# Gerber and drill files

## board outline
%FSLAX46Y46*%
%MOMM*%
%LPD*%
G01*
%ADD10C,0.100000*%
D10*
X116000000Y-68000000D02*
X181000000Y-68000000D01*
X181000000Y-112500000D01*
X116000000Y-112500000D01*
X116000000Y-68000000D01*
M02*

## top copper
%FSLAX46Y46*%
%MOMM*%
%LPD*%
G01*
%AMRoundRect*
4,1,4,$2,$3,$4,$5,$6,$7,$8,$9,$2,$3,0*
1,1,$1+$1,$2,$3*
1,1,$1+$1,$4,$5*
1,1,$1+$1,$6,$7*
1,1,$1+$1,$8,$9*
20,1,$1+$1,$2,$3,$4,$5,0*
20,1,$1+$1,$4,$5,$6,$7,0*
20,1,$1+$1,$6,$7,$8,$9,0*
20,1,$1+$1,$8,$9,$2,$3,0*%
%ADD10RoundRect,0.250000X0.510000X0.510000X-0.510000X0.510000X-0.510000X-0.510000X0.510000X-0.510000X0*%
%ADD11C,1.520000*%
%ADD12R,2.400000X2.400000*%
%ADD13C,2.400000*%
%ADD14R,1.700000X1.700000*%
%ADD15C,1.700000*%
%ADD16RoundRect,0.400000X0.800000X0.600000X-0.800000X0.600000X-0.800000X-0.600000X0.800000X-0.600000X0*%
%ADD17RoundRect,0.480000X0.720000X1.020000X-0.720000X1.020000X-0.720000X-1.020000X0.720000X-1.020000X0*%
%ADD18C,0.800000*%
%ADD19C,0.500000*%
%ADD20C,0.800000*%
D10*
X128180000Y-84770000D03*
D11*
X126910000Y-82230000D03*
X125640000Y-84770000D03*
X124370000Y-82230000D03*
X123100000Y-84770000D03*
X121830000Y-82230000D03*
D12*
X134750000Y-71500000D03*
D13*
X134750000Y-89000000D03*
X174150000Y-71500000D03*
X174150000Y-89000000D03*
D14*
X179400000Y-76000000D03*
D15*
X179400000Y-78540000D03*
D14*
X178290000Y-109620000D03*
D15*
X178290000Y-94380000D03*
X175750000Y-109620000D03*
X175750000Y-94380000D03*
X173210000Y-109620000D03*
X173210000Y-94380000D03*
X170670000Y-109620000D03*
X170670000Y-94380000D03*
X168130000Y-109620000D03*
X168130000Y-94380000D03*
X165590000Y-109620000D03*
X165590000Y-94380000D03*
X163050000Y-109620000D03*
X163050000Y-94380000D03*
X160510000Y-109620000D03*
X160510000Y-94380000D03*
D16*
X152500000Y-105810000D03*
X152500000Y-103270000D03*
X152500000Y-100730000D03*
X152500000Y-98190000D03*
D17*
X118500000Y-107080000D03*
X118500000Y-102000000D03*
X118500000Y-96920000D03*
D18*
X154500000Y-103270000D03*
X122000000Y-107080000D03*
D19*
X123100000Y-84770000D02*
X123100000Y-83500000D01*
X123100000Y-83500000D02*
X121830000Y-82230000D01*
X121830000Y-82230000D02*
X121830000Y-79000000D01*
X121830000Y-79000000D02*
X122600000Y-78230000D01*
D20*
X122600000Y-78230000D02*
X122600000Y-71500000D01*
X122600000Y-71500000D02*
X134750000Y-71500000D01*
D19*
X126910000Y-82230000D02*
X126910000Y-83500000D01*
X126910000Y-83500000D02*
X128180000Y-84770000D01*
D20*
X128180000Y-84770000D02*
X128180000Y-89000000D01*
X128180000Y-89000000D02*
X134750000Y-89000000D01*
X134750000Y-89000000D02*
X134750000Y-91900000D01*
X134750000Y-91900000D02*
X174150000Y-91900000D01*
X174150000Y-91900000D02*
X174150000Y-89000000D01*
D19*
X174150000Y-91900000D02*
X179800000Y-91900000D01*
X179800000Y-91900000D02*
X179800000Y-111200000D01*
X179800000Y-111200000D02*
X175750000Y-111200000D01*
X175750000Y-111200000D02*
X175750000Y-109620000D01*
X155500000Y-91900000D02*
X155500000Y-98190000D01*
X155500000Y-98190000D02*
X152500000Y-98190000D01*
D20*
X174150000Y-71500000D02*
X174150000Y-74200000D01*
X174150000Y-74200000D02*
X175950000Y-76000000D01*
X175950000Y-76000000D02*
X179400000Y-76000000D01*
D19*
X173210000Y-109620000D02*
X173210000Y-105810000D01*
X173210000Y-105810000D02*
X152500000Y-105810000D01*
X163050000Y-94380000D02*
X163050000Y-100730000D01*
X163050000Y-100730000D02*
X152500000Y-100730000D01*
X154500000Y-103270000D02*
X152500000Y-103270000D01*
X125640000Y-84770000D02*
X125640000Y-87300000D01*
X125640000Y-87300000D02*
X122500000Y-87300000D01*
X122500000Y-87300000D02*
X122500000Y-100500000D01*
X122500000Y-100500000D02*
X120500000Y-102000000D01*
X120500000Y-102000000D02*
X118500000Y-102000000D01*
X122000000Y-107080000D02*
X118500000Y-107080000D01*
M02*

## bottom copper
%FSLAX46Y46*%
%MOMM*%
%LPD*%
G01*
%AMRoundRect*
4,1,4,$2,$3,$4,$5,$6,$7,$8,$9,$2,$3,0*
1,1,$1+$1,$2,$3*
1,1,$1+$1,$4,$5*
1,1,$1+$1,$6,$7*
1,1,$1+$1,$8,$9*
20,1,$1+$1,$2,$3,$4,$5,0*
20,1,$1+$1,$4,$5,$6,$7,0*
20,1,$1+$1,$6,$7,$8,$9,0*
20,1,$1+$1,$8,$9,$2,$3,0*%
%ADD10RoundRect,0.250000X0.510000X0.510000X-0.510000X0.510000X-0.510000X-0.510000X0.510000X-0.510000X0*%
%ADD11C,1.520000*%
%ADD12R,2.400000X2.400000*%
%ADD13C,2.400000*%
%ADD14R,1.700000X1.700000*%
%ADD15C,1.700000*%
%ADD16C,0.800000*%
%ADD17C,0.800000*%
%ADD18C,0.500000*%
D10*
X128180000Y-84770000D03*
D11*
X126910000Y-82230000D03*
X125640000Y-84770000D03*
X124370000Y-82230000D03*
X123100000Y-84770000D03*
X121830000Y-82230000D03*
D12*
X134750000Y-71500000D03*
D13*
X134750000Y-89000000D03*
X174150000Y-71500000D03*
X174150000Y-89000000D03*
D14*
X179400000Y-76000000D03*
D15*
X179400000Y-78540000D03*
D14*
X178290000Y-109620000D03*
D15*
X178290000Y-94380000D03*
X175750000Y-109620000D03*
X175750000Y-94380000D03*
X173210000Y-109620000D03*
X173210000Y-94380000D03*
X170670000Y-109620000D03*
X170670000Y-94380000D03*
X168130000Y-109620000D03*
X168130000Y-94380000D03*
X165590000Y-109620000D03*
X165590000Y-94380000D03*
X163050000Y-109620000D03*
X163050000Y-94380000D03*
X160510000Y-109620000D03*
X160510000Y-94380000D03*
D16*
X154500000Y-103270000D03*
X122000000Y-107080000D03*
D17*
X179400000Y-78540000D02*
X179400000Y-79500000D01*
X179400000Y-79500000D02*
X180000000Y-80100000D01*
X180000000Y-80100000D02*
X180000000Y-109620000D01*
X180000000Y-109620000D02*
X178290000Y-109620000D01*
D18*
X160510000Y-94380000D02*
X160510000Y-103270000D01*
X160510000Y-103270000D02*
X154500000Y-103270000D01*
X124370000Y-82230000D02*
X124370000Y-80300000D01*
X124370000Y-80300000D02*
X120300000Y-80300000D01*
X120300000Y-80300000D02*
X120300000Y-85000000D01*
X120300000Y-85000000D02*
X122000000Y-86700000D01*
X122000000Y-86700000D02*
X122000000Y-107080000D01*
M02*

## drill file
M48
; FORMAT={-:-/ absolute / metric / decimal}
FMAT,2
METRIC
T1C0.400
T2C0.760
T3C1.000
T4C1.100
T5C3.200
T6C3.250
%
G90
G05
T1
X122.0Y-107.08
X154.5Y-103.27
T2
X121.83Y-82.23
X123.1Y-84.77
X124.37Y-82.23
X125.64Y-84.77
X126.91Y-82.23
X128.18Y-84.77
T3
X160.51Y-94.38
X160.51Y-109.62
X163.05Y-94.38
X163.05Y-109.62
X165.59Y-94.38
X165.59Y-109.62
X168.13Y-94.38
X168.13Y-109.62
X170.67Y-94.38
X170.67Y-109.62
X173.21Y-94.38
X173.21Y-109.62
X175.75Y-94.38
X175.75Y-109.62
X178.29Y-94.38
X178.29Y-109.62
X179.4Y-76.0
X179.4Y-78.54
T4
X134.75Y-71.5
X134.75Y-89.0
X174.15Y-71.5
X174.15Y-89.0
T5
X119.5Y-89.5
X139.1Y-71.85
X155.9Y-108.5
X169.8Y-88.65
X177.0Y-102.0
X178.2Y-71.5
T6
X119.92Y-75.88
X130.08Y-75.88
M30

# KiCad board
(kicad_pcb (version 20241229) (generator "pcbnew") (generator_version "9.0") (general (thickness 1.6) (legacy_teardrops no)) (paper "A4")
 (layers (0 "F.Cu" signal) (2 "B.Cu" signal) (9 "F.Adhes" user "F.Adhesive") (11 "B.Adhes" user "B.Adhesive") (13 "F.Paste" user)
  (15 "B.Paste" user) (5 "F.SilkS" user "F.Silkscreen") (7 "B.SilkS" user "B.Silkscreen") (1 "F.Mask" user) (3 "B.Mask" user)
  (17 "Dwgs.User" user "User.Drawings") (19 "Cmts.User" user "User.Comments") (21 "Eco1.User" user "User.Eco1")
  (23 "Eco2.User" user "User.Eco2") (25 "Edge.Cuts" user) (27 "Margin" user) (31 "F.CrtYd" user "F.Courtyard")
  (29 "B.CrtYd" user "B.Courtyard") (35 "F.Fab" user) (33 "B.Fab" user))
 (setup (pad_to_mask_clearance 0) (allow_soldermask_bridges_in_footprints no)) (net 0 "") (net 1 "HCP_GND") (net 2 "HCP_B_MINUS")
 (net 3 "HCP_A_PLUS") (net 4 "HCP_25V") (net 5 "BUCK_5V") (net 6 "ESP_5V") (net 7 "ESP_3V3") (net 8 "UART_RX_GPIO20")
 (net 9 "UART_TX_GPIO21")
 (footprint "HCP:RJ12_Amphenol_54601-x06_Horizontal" (layer "F.Cu") (at 128.18 84.77 180)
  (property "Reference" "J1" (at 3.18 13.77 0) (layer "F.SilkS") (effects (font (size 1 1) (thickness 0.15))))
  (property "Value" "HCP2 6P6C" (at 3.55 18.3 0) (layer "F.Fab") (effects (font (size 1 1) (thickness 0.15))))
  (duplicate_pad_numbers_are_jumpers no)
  (pad "" np_thru_hole circle (at -1.9 8.89 180) (size 3.25 3.25) (drill 3.25) (layers "*.Cu" "*.Mask"))
  (pad "" np_thru_hole circle (at 8.26 8.89 180) (size 3.25 3.25) (drill 3.25) (layers "*.Cu" "*.Mask"))
  (pad "1" thru_hole roundrect (at 0 0 180) (size 1.52 1.52) (drill 0.76) (layers "*.Cu" "*.Mask") (remove_unused_layers no)
   (roundrect_rratio 0.1644736842) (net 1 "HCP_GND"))
  (pad "2" thru_hole circle (at 1.27 2.54 180) (size 1.52 1.52) (drill 0.76) (layers "*.Cu" "*.Mask") (remove_unused_layers no)
   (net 1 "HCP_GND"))
  (pad "3" thru_hole circle (at 2.54 0 180) (size 1.52 1.52) (drill 0.76) (layers "*.Cu" "*.Mask") (remove_unused_layers no)
   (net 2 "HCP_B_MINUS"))
  (pad "4" thru_hole circle (at 3.81 2.54 180) (size 1.52 1.52) (drill 0.76) (layers "*.Cu" "*.Mask") (remove_unused_layers no)
   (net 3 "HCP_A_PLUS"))
  (pad "5" thru_hole circle (at 5.08 0 180) (size 1.52 1.52) (drill 0.76) (layers "*.Cu" "*.Mask") (remove_unused_layers no)
   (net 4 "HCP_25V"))
  (pad "6" thru_hole circle (at 6.35 2.54 180) (size 1.52 1.52) (drill 0.76) (layers "*.Cu" "*.Mask") (remove_unused_layers no)
   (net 4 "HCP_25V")))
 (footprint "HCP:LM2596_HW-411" (layer "F.Cu") (at 154.45 80.25 0)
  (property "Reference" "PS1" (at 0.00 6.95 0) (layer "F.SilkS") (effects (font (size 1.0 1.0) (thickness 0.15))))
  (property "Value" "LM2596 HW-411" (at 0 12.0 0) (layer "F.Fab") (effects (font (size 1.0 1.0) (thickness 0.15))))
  (pad "1" thru_hole rect (at -19.7 -8.75) (size 2.4 2.4) (drill 1.1) (layers "*.Cu" "*.Mask") (remove_unused_layers no) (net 4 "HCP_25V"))
  (pad "2" thru_hole circle (at -19.7 8.75) (size 2.4 2.4) (drill 1.1) (layers "*.Cu" "*.Mask") (remove_unused_layers no) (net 1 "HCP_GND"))
  (pad "3" thru_hole circle (at 19.7 -8.75) (size 2.4 2.4) (drill 1.1) (layers "*.Cu" "*.Mask") (remove_unused_layers no) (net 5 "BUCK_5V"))
  (pad "4" thru_hole circle (at 19.7 8.75) (size 2.4 2.4) (drill 1.1) (layers "*.Cu" "*.Mask") (remove_unused_layers no) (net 1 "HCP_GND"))
  (pad "" np_thru_hole circle (at -15.35 -8.4) (size 3.2 3.2) (drill 3.2) (layers "*.Cu" "*.Mask"))
  (pad "" np_thru_hole circle (at 15.35 8.4) (size 3.2 3.2) (drill 3.2) (layers "*.Cu" "*.Mask")))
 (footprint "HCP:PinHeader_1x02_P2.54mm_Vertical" (layer "F.Cu") (at 179.4 76.0 0)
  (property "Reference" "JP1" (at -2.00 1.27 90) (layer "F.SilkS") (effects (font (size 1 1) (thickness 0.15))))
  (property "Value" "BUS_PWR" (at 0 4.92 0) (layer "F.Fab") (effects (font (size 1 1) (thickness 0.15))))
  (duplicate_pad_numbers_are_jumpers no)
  (pad "1" thru_hole rect (at 0 0) (size 1.7 1.7) (drill 1) (layers "*.Cu" "*.Mask") (remove_unused_layers no) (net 5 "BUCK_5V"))
  (pad "2" thru_hole circle (at 0 2.54) (size 1.7 1.7) (drill 1) (layers "*.Cu" "*.Mask") (remove_unused_layers no) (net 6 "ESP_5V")))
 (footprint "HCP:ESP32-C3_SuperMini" (layer "F.Cu") (at 169.4 102.0 270)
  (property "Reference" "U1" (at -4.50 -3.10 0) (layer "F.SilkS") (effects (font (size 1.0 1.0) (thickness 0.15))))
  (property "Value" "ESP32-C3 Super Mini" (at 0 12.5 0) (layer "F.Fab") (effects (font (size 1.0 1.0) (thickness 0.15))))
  (pad "1" thru_hole rect (at 7.62 -8.89 270) (size 1.7 1.7) (drill 1.0) (layers "*.Cu" "*.Mask") (remove_unused_layers no) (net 6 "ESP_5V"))
  (pad "2" thru_hole circle (at -7.62 -8.89 270) (size 1.7 1.7) (drill 1.0) (layers "*.Cu" "*.Mask") (remove_unused_layers no))
  (pad "3" thru_hole circle (at 7.62 -6.35 270) (size 1.7 1.7) (drill 1.0) (layers "*.Cu" "*.Mask") (remove_unused_layers no)
   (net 1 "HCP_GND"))
  (pad "4" thru_hole circle (at -7.62 -6.35 270) (size 1.7 1.7) (drill 1.0) (layers "*.Cu" "*.Mask") (remove_unused_layers no))
  (pad "5" thru_hole circle (at 7.62 -3.81 270) (size 1.7 1.7) (drill 1.0) (layers "*.Cu" "*.Mask") (remove_unused_layers no)
   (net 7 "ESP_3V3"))
  (pad "6" thru_hole circle (at -7.62 -3.81 270) (size 1.7 1.7) (drill 1.0) (layers "*.Cu" "*.Mask") (remove_unused_layers no))
  (pad "7" thru_hole circle (at 7.62 -1.27 270) (size 1.7 1.7) (drill 1.0) (layers "*.Cu" "*.Mask") (remove_unused_layers no))
  (pad "8" thru_hole circle (at -7.62 -1.27 270) (size 1.7 1.7) (drill 1.0) (layers "*.Cu" "*.Mask") (remove_unused_layers no))
  (pad "9" thru_hole circle (at 7.62 1.27 270) (size 1.7 1.7) (drill 1.0) (layers "*.Cu" "*.Mask") (remove_unused_layers no))
  (pad "10" thru_hole circle (at -7.62 1.27 270) (size 1.7 1.7) (drill 1.0) (layers "*.Cu" "*.Mask") (remove_unused_layers no))
  (pad "11" thru_hole circle (at 7.62 3.81 270) (size 1.7 1.7) (drill 1.0) (layers "*.Cu" "*.Mask") (remove_unused_layers no))
  (pad "12" thru_hole circle (at -7.62 3.81 270) (size 1.7 1.7) (drill 1.0) (layers "*.Cu" "*.Mask") (remove_unused_layers no))
  (pad "13" thru_hole circle (at 7.62 6.35 270) (size 1.7 1.7) (drill 1.0) (layers "*.Cu" "*.Mask") (remove_unused_layers no))
  (pad "14" thru_hole circle (at -7.62 6.35 270) (size 1.7 1.7) (drill 1.0) (layers "*.Cu" "*.Mask") (remove_unused_layers no)
   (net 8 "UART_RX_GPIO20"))
  (pad "15" thru_hole circle (at 7.62 8.89 270) (size 1.7 1.7) (drill 1.0) (layers "*.Cu" "*.Mask") (remove_unused_layers no))
  (pad "16" thru_hole circle (at -7.62 8.89 270) (size 1.7 1.7) (drill 1.0) (layers "*.Cu" "*.Mask") (remove_unused_layers no)
   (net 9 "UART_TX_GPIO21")))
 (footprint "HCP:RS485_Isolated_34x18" (layer "F.Cu") (at 135.5 102.0 180)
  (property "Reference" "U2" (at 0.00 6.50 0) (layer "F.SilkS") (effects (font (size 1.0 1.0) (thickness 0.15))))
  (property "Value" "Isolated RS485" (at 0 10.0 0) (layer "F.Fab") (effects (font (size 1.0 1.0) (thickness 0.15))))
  (pad "1" smd roundrect (at -17 -3.81 180) (size 2.4 2.0) (layers "F.Cu" "F.Paste" "F.Mask") (roundrect_rratio 0.2) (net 7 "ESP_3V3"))
  (pad "2" smd roundrect (at -17 -1.27 180) (size 2.4 2.0) (layers "F.Cu" "F.Paste" "F.Mask") (roundrect_rratio 0.2)
   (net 9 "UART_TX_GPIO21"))
  (pad "3" smd roundrect (at -17 1.27 180) (size 2.4 2.0) (layers "F.Cu" "F.Paste" "F.Mask") (roundrect_rratio 0.2) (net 8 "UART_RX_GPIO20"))
  (pad "4" smd roundrect (at -17 3.81 180) (size 2.4 2.0) (layers "F.Cu" "F.Paste" "F.Mask") (roundrect_rratio 0.2) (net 1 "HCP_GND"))
  (pad "5" smd roundrect (at 17 -5.08 180) (size 2.4 3.0) (layers "F.Cu" "F.Paste" "F.Mask") (roundrect_rratio 0.2) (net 3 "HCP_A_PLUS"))
  (pad "6" smd roundrect (at 17 0 180) (size 2.4 3.0) (layers "F.Cu" "F.Paste" "F.Mask") (roundrect_rratio 0.2) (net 2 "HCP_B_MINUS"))
  (pad "7" smd roundrect (at 17 5.08 180) (size 2.4 3.0) (layers "F.Cu" "F.Paste" "F.Mask") (roundrect_rratio 0.2)))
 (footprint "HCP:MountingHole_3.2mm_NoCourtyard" (layer "F.Cu") (at 119.5 89.5 0)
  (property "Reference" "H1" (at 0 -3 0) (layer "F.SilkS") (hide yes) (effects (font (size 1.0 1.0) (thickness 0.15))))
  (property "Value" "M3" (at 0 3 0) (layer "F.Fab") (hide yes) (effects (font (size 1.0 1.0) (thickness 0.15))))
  (pad "" np_thru_hole circle (at 0 0) (size 3.2 3.2) (drill 3.2) (layers "*.Cu" "*.Mask")))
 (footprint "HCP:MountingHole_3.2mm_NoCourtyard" (layer "F.Cu") (at 178.2 71.5 0)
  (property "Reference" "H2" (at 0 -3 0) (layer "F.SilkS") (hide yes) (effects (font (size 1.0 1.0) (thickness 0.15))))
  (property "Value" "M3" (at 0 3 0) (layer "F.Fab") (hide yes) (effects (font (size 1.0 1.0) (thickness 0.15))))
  (pad "" np_thru_hole circle (at 0 0) (size 3.2 3.2) (drill 3.2) (layers "*.Cu" "*.Mask")))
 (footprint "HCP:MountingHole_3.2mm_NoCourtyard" (layer "F.Cu") (at 155.9 108.5 0)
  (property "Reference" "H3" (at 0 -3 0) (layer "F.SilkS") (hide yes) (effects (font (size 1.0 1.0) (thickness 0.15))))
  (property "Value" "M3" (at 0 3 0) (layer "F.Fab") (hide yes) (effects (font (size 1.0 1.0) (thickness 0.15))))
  (pad "" np_thru_hole circle (at 0 0) (size 3.2 3.2) (drill 3.2) (layers "*.Cu" "*.Mask")))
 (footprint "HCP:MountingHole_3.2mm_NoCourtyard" (layer "F.Cu") (at 177.0 102.0 0)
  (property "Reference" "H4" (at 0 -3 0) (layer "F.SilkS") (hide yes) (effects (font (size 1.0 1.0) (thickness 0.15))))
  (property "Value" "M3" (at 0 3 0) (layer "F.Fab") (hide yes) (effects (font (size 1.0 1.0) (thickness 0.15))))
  (pad "" np_thru_hole circle (at 0 0) (size 3.2 3.2) (drill 3.2) (layers "*.Cu" "*.Mask")))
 (segment (start 123.1 84.77) (end 123.1 83.5) (width 0.5) (layer "F.Cu") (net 4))
 (segment (start 123.1 83.5) (end 121.83 82.23) (width 0.5) (layer "F.Cu") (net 4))
 (segment (start 121.83 82.23) (end 121.83 79.0) (width 0.5) (layer "F.Cu") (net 4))
 (segment (start 121.83 79.0) (end 122.6 78.23) (width 0.5) (layer "F.Cu") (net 4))
 (segment (start 122.6 78.23) (end 122.6 71.5) (width 0.8) (layer "F.Cu") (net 4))
 (segment (start 122.6 71.5) (end 134.75 71.5) (width 0.8) (layer "F.Cu") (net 4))
 (segment (start 126.91 82.23) (end 126.91 83.5) (width 0.5) (layer "F.Cu") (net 1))
 (segment (start 126.91 83.5) (end 128.18 84.77) (width 0.5) (layer "F.Cu") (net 1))
 (segment (start 128.18 84.77) (end 128.18 89.0) (width 0.8) (layer "F.Cu") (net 1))
 (segment (start 128.18 89.0) (end 134.75 89.0) (width 0.8) (layer "F.Cu") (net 1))
 (segment (start 134.75 89.0) (end 134.75 91.9) (width 0.8) (layer "F.Cu") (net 1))
 (segment (start 134.75 91.9) (end 174.15 91.9) (width 0.8) (layer "F.Cu") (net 1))
 (segment (start 174.15 91.9) (end 174.15 89.0) (width 0.8) (layer "F.Cu") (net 1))
 (segment (start 174.15 91.9) (end 179.8 91.9) (width 0.5) (layer "F.Cu") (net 1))
 (segment (start 179.8 91.9) (end 179.8 111.2) (width 0.5) (layer "F.Cu") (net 1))
 (segment (start 179.8 111.2) (end 175.75 111.2) (width 0.5) (layer "F.Cu") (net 1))
 (segment (start 175.75 111.2) (end 175.75 109.62) (width 0.5) (layer "F.Cu") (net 1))
 (segment (start 155.5 91.9) (end 155.5 98.19) (width 0.5) (layer "F.Cu") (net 1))
 (segment (start 155.5 98.19) (end 152.5 98.19) (width 0.5) (layer "F.Cu") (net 1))
 (segment (start 174.15 71.5) (end 174.15 74.2) (width 0.8) (layer "F.Cu") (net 5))
 (segment (start 174.15 74.2) (end 175.95 76.0) (width 0.8) (layer "F.Cu") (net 5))
 (segment (start 175.95 76.0) (end 179.4 76.0) (width 0.8) (layer "F.Cu") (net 5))
 (segment (start 179.4 78.54) (end 179.4 79.5) (width 0.8) (layer "B.Cu") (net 6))
 (segment (start 179.4 79.5) (end 180.0 80.1) (width 0.8) (layer "B.Cu") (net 6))
 (segment (start 180.0 80.1) (end 180.0 109.62) (width 0.8) (layer "B.Cu") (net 6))
 (segment (start 180.0 109.62) (end 178.29 109.62) (width 0.8) (layer "B.Cu") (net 6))
 (segment (start 173.21 109.62) (end 173.21 105.81) (width 0.5) (layer "F.Cu") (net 7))
 (segment (start 173.21 105.81) (end 152.5 105.81) (width 0.5) (layer "F.Cu") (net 7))
 (segment (start 163.05 94.38) (end 163.05 100.73) (width 0.5) (layer "F.Cu") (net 8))
 (segment (start 163.05 100.73) (end 152.5 100.73) (width 0.5) (layer "F.Cu") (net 8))
 (segment (start 160.51 94.38) (end 160.51 103.27) (width 0.5) (layer "B.Cu") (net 9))
 (segment (start 160.51 103.27) (end 154.5 103.27) (width 0.5) (layer "B.Cu") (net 9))
 (segment (start 154.5 103.27) (end 152.5 103.27) (width 0.5) (layer "F.Cu") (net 9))
 (segment (start 125.64 84.77) (end 125.64 87.3) (width 0.5) (layer "F.Cu") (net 2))
 (segment (start 125.64 87.3) (end 122.5 87.3) (width 0.5) (layer "F.Cu") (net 2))
 (segment (start 122.5 87.3) (end 122.5 100.5) (width 0.5) (layer "F.Cu") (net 2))
 (segment (start 122.5 100.5) (end 120.5 102.0) (width 0.5) (layer "F.Cu") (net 2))
 (segment (start 120.5 102.0) (end 118.5 102.0) (width 0.5) (layer "F.Cu") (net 2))
 (segment (start 124.37 82.23) (end 124.37 80.3) (width 0.5) (layer "B.Cu") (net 3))
 (segment (start 124.37 80.3) (end 120.3 80.3) (width 0.5) (layer "B.Cu") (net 3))
 (segment (start 120.3 80.3) (end 120.3 85.0) (width 0.5) (layer "B.Cu") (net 3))
 (segment (start 120.3 85.0) (end 122.0 86.7) (width 0.5) (layer "B.Cu") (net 3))
 (segment (start 122.0 86.7) (end 122.0 107.08) (width 0.5) (layer "B.Cu") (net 3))
 (segment (start 122.0 107.08) (end 118.5 107.08) (width 0.5) (layer "F.Cu") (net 3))
 (via (at 154.5 103.27) (size 0.8) (drill 0.4) (layers "F.Cu" "B.Cu") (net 9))
 (via (at 122.0 107.08) (size 0.8) (drill 0.4) (layers "F.Cu" "B.Cu") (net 3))
 (gr_rect (start 116.0 68.0) (end 181.0 112.5) (stroke (width 0.1) (type default)) (fill none) (layer "Edge.Cuts")))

